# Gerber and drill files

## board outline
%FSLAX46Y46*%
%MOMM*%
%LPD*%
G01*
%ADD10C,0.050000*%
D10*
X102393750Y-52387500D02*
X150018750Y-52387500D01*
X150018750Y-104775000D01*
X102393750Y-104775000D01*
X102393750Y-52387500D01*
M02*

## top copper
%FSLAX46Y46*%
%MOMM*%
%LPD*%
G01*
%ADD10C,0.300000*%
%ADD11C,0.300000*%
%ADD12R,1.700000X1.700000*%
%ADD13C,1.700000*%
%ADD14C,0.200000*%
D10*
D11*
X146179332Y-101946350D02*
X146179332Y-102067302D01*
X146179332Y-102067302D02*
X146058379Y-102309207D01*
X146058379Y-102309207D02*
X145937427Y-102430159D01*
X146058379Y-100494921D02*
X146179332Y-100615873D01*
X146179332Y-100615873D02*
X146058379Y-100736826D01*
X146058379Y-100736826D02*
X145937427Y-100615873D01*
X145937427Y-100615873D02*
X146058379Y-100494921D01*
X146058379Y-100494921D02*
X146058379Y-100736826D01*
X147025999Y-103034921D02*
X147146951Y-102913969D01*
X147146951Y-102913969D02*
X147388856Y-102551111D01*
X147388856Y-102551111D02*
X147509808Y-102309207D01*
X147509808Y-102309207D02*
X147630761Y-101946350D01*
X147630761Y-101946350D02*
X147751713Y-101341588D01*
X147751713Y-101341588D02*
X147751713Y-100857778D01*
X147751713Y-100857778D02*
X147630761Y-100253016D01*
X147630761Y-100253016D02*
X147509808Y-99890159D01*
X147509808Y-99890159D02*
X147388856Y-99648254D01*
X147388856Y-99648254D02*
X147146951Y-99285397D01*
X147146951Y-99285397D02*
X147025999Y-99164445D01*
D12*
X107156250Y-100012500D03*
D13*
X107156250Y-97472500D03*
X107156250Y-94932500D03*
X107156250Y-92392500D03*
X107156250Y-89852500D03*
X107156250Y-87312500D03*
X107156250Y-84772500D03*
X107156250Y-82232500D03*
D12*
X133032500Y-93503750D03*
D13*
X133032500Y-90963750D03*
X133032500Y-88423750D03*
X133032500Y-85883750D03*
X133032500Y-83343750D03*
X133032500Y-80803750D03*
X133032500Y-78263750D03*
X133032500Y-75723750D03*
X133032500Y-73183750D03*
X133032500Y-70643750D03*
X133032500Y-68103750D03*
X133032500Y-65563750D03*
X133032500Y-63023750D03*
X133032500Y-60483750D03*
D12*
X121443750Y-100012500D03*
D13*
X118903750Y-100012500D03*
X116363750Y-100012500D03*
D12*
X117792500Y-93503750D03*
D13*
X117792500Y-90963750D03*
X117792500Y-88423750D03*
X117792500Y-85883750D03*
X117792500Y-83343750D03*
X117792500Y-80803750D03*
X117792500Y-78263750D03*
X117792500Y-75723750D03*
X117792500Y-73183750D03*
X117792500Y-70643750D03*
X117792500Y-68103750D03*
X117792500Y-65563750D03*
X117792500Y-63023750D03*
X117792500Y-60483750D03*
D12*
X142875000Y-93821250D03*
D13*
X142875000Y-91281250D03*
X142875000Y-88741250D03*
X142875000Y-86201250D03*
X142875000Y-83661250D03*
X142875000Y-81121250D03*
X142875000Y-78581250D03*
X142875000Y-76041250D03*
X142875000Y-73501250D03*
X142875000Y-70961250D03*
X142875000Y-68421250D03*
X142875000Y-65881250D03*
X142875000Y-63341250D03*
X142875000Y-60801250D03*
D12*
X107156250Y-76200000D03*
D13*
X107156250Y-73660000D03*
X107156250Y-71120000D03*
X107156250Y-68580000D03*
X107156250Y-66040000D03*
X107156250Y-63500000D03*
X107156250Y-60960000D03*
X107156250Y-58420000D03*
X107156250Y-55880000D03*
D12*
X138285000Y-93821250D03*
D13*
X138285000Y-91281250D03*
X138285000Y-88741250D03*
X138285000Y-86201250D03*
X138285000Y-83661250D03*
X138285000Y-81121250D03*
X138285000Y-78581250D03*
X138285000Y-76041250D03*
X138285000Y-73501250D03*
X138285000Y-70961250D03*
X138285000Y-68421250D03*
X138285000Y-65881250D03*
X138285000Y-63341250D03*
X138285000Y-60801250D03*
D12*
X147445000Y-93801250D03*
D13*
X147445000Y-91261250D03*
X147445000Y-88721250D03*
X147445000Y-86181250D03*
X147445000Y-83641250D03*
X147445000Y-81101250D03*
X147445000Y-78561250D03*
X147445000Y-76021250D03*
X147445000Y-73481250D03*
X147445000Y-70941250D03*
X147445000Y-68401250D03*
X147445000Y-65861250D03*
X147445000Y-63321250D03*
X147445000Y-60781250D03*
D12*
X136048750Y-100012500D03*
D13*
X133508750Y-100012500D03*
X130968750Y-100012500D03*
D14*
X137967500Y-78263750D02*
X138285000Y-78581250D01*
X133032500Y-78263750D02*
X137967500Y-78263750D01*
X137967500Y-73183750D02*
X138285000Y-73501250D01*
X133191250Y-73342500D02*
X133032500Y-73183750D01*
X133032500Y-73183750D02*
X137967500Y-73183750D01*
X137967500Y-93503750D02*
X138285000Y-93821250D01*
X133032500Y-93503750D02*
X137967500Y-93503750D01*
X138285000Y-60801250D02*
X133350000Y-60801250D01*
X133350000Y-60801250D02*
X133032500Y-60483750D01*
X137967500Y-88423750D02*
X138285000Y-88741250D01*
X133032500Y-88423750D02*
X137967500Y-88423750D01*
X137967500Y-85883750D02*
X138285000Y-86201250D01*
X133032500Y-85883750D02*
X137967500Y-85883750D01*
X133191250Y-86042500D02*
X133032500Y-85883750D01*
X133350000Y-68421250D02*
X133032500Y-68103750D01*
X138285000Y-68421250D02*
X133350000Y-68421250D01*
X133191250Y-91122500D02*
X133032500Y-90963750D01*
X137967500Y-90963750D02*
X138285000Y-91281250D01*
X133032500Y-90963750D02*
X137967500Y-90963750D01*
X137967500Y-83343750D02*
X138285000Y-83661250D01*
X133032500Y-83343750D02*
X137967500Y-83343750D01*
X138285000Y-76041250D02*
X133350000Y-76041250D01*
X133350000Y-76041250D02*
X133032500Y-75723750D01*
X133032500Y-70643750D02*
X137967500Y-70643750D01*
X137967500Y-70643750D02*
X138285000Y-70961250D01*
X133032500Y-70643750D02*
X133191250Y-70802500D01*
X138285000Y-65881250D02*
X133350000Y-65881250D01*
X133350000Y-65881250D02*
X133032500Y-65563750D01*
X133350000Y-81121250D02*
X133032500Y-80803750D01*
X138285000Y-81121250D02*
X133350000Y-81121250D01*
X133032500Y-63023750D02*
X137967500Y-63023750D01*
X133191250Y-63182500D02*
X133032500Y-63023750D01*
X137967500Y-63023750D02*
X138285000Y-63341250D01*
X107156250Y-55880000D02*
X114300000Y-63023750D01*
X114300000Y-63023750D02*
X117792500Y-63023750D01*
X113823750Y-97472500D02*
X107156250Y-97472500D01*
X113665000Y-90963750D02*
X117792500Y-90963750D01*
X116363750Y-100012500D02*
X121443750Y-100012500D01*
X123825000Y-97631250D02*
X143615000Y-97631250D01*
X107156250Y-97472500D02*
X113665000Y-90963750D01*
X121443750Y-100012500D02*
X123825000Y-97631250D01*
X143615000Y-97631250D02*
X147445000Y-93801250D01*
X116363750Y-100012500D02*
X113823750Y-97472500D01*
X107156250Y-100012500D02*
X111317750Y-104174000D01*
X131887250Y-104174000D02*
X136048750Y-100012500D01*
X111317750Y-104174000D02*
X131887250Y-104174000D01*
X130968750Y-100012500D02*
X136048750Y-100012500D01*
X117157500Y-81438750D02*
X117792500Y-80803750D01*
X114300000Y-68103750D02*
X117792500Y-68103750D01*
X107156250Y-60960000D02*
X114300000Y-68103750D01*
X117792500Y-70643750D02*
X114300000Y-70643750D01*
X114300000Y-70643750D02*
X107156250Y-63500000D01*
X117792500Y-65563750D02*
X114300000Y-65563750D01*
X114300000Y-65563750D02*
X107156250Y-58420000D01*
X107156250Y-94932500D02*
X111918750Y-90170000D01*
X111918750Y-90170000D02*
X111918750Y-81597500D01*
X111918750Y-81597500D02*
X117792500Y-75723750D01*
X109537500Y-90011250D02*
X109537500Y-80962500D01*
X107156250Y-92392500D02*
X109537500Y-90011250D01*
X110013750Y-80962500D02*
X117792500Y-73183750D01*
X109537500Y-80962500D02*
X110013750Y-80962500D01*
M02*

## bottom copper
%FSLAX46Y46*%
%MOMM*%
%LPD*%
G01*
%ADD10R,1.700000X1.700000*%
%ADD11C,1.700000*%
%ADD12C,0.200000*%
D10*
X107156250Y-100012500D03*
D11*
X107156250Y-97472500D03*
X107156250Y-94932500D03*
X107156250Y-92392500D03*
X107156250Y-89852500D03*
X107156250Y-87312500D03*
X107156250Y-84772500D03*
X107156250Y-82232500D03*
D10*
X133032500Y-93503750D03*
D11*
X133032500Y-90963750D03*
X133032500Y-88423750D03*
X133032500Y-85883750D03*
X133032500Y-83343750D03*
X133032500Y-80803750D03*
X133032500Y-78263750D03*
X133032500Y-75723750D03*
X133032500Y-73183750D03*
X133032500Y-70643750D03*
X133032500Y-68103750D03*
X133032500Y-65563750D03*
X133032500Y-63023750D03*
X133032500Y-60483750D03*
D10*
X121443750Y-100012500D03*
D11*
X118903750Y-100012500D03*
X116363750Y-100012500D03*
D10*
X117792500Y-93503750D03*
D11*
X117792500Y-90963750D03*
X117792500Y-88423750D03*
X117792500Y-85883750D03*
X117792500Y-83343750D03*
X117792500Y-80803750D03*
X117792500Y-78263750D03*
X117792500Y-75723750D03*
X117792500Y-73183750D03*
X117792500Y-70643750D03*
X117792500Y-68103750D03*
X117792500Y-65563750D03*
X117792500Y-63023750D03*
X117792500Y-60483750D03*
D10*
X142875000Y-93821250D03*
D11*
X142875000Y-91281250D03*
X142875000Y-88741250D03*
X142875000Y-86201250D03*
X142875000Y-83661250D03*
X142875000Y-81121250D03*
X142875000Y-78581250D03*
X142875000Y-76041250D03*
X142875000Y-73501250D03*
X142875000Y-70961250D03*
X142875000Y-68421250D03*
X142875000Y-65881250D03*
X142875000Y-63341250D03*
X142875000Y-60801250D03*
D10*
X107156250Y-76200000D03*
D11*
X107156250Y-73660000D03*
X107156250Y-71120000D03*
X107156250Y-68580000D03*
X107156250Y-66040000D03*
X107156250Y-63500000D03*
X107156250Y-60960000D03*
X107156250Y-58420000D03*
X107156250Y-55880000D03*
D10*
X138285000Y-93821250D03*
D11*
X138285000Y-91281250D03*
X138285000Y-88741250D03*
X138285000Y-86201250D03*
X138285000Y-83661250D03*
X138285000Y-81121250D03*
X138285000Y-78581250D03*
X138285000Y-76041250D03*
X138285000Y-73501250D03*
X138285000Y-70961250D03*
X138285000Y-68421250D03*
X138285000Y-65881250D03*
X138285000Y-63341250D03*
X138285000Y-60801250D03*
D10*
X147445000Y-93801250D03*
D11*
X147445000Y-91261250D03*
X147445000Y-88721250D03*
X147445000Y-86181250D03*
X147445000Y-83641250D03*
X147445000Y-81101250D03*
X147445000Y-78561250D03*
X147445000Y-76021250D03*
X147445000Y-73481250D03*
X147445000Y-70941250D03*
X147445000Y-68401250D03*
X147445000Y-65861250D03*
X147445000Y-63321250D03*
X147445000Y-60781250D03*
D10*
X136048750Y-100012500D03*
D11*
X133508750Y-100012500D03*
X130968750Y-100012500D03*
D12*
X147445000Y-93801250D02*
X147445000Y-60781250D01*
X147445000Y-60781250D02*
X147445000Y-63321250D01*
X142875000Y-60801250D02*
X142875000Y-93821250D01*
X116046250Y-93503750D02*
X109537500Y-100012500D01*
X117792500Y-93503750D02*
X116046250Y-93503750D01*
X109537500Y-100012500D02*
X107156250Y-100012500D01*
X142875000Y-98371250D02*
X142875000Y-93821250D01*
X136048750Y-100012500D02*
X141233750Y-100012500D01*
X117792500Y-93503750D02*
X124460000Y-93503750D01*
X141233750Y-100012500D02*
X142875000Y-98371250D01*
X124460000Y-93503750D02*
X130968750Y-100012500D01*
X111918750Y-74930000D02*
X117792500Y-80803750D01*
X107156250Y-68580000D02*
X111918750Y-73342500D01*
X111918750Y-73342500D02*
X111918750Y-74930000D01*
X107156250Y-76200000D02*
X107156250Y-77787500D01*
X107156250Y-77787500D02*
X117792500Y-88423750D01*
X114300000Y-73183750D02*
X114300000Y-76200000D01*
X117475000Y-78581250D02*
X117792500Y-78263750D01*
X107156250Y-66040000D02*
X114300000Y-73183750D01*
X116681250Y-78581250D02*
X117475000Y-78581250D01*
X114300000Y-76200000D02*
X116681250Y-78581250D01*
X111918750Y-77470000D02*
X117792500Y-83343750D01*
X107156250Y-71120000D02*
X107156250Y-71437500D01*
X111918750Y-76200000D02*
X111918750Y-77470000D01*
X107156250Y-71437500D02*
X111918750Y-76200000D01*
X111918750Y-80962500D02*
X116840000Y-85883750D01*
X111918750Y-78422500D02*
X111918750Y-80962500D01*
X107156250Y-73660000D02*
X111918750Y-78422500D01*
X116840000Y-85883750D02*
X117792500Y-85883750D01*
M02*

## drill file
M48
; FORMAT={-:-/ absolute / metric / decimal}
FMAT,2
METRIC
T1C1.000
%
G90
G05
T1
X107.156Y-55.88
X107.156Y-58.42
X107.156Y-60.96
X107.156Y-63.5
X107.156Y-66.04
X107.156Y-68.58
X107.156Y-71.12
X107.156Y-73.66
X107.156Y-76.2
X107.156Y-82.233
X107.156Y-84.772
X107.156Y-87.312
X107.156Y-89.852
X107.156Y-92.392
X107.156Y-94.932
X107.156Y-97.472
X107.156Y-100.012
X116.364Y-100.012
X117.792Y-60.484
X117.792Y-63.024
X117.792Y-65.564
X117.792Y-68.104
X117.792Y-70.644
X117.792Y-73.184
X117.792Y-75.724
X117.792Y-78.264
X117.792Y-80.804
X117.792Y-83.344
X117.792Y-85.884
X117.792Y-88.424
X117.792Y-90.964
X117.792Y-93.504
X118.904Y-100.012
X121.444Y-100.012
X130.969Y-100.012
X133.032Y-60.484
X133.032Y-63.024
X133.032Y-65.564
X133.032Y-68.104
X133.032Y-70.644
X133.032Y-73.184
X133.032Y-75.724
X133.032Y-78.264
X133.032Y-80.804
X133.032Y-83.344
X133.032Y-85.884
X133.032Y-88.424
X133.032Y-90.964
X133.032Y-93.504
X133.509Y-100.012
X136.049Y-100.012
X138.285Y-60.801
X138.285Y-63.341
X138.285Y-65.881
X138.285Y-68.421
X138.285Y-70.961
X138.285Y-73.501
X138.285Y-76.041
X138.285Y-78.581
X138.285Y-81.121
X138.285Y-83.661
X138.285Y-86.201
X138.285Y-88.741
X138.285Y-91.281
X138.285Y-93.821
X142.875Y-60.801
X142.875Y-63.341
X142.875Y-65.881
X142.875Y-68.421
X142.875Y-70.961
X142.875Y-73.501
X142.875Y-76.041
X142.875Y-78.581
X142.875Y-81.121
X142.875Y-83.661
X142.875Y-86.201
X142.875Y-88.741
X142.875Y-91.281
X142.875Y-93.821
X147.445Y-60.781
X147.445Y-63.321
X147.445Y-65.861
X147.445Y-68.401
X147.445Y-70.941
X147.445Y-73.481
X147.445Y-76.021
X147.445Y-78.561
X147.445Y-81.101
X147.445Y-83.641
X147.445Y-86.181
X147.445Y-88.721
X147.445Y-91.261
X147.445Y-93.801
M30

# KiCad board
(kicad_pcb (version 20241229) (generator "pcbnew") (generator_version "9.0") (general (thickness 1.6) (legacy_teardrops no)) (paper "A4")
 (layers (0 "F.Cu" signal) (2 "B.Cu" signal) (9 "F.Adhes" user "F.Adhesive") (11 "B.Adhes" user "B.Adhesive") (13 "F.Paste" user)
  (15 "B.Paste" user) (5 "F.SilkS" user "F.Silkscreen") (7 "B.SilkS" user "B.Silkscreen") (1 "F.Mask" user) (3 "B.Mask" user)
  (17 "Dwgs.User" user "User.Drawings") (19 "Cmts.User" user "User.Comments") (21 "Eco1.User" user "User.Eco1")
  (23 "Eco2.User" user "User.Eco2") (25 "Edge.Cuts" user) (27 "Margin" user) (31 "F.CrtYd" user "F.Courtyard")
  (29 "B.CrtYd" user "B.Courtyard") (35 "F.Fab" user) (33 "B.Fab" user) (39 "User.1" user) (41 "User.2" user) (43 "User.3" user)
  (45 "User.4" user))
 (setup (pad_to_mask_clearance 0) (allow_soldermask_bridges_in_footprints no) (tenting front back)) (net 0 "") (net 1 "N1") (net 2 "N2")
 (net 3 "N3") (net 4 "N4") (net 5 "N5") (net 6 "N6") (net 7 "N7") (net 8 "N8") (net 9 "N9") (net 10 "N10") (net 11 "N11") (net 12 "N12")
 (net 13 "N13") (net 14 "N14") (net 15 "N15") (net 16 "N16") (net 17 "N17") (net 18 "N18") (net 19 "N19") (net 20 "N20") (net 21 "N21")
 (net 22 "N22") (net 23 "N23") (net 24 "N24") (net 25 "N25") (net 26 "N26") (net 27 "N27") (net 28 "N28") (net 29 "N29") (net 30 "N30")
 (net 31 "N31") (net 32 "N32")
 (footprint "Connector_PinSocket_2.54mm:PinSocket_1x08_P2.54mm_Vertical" (layer "F.Cu") (at 107.15625 100.0125 180)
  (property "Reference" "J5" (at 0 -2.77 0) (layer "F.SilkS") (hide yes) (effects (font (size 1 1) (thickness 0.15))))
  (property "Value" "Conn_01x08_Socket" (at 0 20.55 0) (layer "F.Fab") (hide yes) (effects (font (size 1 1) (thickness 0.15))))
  (pad "1" thru_hole rect (at 0 0 180) (size 1.7 1.7) (drill 1) (layers "*.Cu" "*.Mask") (remove_unused_layers no) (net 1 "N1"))
  (pad "2" thru_hole circle (at 0 2.54 180) (size 1.7 1.7) (drill 1) (layers "*.Cu" "*.Mask") (remove_unused_layers no) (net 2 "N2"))
  (pad "3" thru_hole circle (at 0 5.08 180) (size 1.7 1.7) (drill 1) (layers "*.Cu" "*.Mask") (remove_unused_layers no) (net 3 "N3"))
  (pad "4" thru_hole circle (at 0 7.62 180) (size 1.7 1.7) (drill 1) (layers "*.Cu" "*.Mask") (remove_unused_layers no) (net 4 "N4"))
  (pad "5" thru_hole circle (at 0 10.16 180) (size 1.7 1.7) (drill 1) (layers "*.Cu" "*.Mask") (remove_unused_layers no) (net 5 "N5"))
  (pad "6" thru_hole circle (at 0 12.7 180) (size 1.7 1.7) (drill 1) (layers "*.Cu" "*.Mask") (remove_unused_layers no) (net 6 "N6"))
  (pad "7" thru_hole circle (at 0 15.24 180) (size 1.7 1.7) (drill 1) (layers "*.Cu" "*.Mask") (remove_unused_layers no) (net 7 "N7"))
  (pad "8" thru_hole circle (at 0 17.78 180) (size 1.7 1.7) (drill 1) (layers "*.Cu" "*.Mask") (remove_unused_layers no) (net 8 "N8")))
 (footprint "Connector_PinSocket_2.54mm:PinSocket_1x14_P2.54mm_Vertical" (layer "F.Cu") (at 133.0325 93.50375 180)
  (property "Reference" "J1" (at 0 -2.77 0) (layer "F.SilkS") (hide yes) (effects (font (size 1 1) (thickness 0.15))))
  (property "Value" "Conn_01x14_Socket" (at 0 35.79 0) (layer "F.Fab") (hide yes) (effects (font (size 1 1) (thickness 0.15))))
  (pad "1" thru_hole rect (at 0 0 180) (size 1.7 1.7) (drill 1) (layers "*.Cu" "*.Mask") (remove_unused_layers no) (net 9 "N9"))
  (pad "2" thru_hole circle (at 0 2.54 180) (size 1.7 1.7) (drill 1) (layers "*.Cu" "*.Mask") (remove_unused_layers no) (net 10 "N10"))
  (pad "3" thru_hole circle (at 0 5.08 180) (size 1.7 1.7) (drill 1) (layers "*.Cu" "*.Mask") (remove_unused_layers no) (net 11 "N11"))
  (pad "4" thru_hole circle (at 0 7.62 180) (size 1.7 1.7) (drill 1) (layers "*.Cu" "*.Mask") (remove_unused_layers no) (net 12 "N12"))
  (pad "5" thru_hole circle (at 0 10.16 180) (size 1.7 1.7) (drill 1) (layers "*.Cu" "*.Mask") (remove_unused_layers no) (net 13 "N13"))
  (pad "6" thru_hole circle (at 0 12.7 180) (size 1.7 1.7) (drill 1) (layers "*.Cu" "*.Mask") (remove_unused_layers no) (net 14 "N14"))
  (pad "7" thru_hole circle (at 0 15.24 180) (size 1.7 1.7) (drill 1) (layers "*.Cu" "*.Mask") (remove_unused_layers no) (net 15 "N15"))
  (pad "8" thru_hole circle (at 0 17.78 180) (size 1.7 1.7) (drill 1) (layers "*.Cu" "*.Mask") (remove_unused_layers no) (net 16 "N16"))
  (pad "9" thru_hole circle (at 0 20.32 180) (size 1.7 1.7) (drill 1) (layers "*.Cu" "*.Mask") (remove_unused_layers no) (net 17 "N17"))
  (pad "10" thru_hole circle (at 0 22.86 180) (size 1.7 1.7) (drill 1) (layers "*.Cu" "*.Mask") (remove_unused_layers no) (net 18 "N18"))
  (pad "11" thru_hole circle (at 0 25.4 180) (size 1.7 1.7) (drill 1) (layers "*.Cu" "*.Mask") (remove_unused_layers no) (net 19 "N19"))
  (pad "12" thru_hole circle (at 0 27.94 180) (size 1.7 1.7) (drill 1) (layers "*.Cu" "*.Mask") (remove_unused_layers no) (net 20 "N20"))
  (pad "13" thru_hole circle (at 0 30.48 180) (size 1.7 1.7) (drill 1) (layers "*.Cu" "*.Mask") (remove_unused_layers no) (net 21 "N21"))
  (pad "14" thru_hole circle (at 0 33.02 180) (size 1.7 1.7) (drill 1) (layers "*.Cu" "*.Mask") (remove_unused_layers no) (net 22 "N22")))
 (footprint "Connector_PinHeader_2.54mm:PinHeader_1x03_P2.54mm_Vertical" (layer "F.Cu") (at 121.44375 100.0125 -90)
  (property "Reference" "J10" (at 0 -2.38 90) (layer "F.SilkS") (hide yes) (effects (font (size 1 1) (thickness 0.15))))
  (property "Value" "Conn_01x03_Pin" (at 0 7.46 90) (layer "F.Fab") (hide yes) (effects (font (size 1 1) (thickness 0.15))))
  (pad "1" thru_hole rect (at 0 0 270) (size 1.7 1.7) (drill 1) (layers "*.Cu" "*.Mask") (remove_unused_layers no) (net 2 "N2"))
  (pad "2" thru_hole circle (at 0 2.54 270) (size 1.7 1.7) (drill 1) (layers "*.Cu" "*.Mask") (remove_unused_layers no) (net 2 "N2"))
  (pad "3" thru_hole circle (at 0 5.08 270) (size 1.7 1.7) (drill 1) (layers "*.Cu" "*.Mask") (remove_unused_layers no) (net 2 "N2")))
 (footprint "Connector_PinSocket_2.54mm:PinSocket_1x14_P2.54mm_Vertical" (layer "F.Cu") (at 117.7925 93.50375 180)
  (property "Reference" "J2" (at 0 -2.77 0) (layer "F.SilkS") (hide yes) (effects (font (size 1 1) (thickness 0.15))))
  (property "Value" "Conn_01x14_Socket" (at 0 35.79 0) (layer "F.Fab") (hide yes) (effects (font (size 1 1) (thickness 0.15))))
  (pad "1" thru_hole rect (at 0 0 180) (size 1.7 1.7) (drill 1) (layers "*.Cu" "*.Mask") (remove_unused_layers no) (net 1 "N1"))
  (pad "2" thru_hole circle (at 0 2.54 180) (size 1.7 1.7) (drill 1) (layers "*.Cu" "*.Mask") (remove_unused_layers no) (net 2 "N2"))
  (pad "3" thru_hole circle (at 0 5.08 180) (size 1.7 1.7) (drill 1) (layers "*.Cu" "*.Mask") (remove_unused_layers no) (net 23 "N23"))
  (pad "4" thru_hole circle (at 0 7.62 180) (size 1.7 1.7) (drill 1) (layers "*.Cu" "*.Mask") (remove_unused_layers no) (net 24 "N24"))
  (pad "5" thru_hole circle (at 0 10.16 180) (size 1.7 1.7) (drill 1) (layers "*.Cu" "*.Mask") (remove_unused_layers no) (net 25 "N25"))
  (pad "6" thru_hole circle (at 0 12.7 180) (size 1.7 1.7) (drill 1) (layers "*.Cu" "*.Mask") (remove_unused_layers no) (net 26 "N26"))
  (pad "7" thru_hole circle (at 0 15.24 180) (size 1.7 1.7) (drill 1) (layers "*.Cu" "*.Mask") (remove_unused_layers no) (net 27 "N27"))
  (pad "8" thru_hole circle (at 0 17.78 180) (size 1.7 1.7) (drill 1) (layers "*.Cu" "*.Mask") (remove_unused_layers no) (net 3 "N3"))
  (pad "9" thru_hole circle (at 0 20.32 180) (size 1.7 1.7) (drill 1) (layers "*.Cu" "*.Mask") (remove_unused_layers no) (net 4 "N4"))
  (pad "10" thru_hole circle (at 0 22.86 180) (size 1.7 1.7) (drill 1) (layers "*.Cu" "*.Mask") (remove_unused_layers no) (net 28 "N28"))
  (pad "11" thru_hole circle (at 0 25.4 180) (size 1.7 1.7) (drill 1) (layers "*.Cu" "*.Mask") (remove_unused_layers no) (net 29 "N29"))
  (pad "12" thru_hole circle (at 0 27.94 180) (size 1.7 1.7) (drill 1) (layers "*.Cu" "*.Mask") (remove_unused_layers no) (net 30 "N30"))
  (pad "13" thru_hole circle (at 0 30.48 180) (size 1.7 1.7) (drill 1) (layers "*.Cu" "*.Mask") (remove_unused_layers no) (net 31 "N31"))
  (pad "14" thru_hole circle (at 0 33.02 180) (size 1.7 1.7) (drill 1) (layers "*.Cu" "*.Mask") (remove_unused_layers no) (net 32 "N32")))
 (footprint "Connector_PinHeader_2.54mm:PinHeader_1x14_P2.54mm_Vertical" (layer "F.Cu") (at 142.875 93.82125 180)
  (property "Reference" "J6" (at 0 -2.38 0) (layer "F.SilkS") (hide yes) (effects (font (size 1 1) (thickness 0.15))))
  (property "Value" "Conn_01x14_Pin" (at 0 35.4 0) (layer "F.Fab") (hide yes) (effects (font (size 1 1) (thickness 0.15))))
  (pad "1" thru_hole rect (at 0 0 180) (size 1.7 1.7) (drill 1) (layers "*.Cu" "*.Mask") (remove_unused_layers no) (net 1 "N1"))
  (pad "2" thru_hole circle (at 0 2.54 180) (size 1.7 1.7) (drill 1) (layers "*.Cu" "*.Mask") (remove_unused_layers no) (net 1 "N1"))
  (pad "3" thru_hole circle (at 0 5.08 180) (size 1.7 1.7) (drill 1) (layers "*.Cu" "*.Mask") (remove_unused_layers no) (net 1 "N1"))
  (pad "4" thru_hole circle (at 0 7.62 180) (size 1.7 1.7) (drill 1) (layers "*.Cu" "*.Mask") (remove_unused_layers no) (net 1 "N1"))
  (pad "5" thru_hole circle (at 0 10.16 180) (size 1.7 1.7) (drill 1) (layers "*.Cu" "*.Mask") (remove_unused_layers no) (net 1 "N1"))
  (pad "6" thru_hole circle (at 0 12.7 180) (size 1.7 1.7) (drill 1) (layers "*.Cu" "*.Mask") (remove_unused_layers no) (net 1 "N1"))
  (pad "7" thru_hole circle (at 0 15.24 180) (size 1.7 1.7) (drill 1) (layers "*.Cu" "*.Mask") (remove_unused_layers no) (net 1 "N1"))
  (pad "8" thru_hole circle (at 0 17.78 180) (size 1.7 1.7) (drill 1) (layers "*.Cu" "*.Mask") (remove_unused_layers no) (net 1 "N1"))
  (pad "9" thru_hole circle (at 0 20.32 180) (size 1.7 1.7) (drill 1) (layers "*.Cu" "*.Mask") (remove_unused_layers no) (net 1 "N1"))
  (pad "10" thru_hole circle (at 0 22.86 180) (size 1.7 1.7) (drill 1) (layers "*.Cu" "*.Mask") (remove_unused_layers no) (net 1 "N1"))
  (pad "11" thru_hole circle (at 0 25.4 180) (size 1.7 1.7) (drill 1) (layers "*.Cu" "*.Mask") (remove_unused_layers no) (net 1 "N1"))
  (pad "12" thru_hole circle (at 0 27.94 180) (size 1.7 1.7) (drill 1) (layers "*.Cu" "*.Mask") (remove_unused_layers no) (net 1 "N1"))
  (pad "13" thru_hole circle (at 0 30.48 180) (size 1.7 1.7) (drill 1) (layers "*.Cu" "*.Mask") (remove_unused_layers no) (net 1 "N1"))
  (pad "14" thru_hole circle (at 0 33.02 180) (size 1.7 1.7) (drill 1) (layers "*.Cu" "*.Mask") (remove_unused_layers no) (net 1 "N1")))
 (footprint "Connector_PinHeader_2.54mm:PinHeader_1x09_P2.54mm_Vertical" (layer "F.Cu") (at 107.15625 76.2 180)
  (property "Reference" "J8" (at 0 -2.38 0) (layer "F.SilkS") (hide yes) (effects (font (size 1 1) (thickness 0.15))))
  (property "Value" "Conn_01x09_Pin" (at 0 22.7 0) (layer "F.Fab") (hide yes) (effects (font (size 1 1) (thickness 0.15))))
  (pad "1" thru_hole rect (at 0 0 180) (size 1.7 1.7) (drill 1) (layers "*.Cu" "*.Mask") (remove_unused_layers no) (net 23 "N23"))
  (pad "2" thru_hole circle (at 0 2.54 180) (size 1.7 1.7) (drill 1) (layers "*.Cu" "*.Mask") (remove_unused_layers no) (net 24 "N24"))
  (pad "3" thru_hole circle (at 0 5.08 180) (size 1.7 1.7) (drill 1) (layers "*.Cu" "*.Mask") (remove_unused_layers no) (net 25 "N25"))
  (pad "4" thru_hole circle (at 0 7.62 180) (size 1.7 1.7) (drill 1) (layers "*.Cu" "*.Mask") (remove_unused_layers no) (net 26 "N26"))
  (pad "5" thru_hole circle (at 0 10.16 180) (size 1.7 1.7) (drill 1) (layers "*.Cu" "*.Mask") (remove_unused_layers no) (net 27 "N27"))
  (pad "6" thru_hole circle (at 0 12.7 180) (size 1.7 1.7) (drill 1) (layers "*.Cu" "*.Mask") (remove_unused_layers no) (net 28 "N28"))
  (pad "7" thru_hole circle (at 0 15.24 180) (size 1.7 1.7) (drill 1) (layers "*.Cu" "*.Mask") (remove_unused_layers no) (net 29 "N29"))
  (pad "8" thru_hole circle (at 0 17.78 180) (size 1.7 1.7) (drill 1) (layers "*.Cu" "*.Mask") (remove_unused_layers no) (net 30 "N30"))
  (pad "9" thru_hole circle (at 0 20.32 180) (size 1.7 1.7) (drill 1) (layers "*.Cu" "*.Mask") (remove_unused_layers no) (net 31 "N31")))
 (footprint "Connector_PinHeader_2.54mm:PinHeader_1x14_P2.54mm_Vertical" (layer "F.Cu") (at 138.285 93.82125 180)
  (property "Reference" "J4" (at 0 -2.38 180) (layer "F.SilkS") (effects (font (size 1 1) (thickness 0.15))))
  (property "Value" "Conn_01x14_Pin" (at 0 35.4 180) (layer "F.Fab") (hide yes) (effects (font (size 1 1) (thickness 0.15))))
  (pad "1" thru_hole rect (at 0 0 180) (size 1.7 1.7) (drill 1) (layers "*.Cu" "*.Mask") (remove_unused_layers no) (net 9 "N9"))
  (pad "2" thru_hole circle (at 0 2.54 180) (size 1.7 1.7) (drill 1) (layers "*.Cu" "*.Mask") (remove_unused_layers no) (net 10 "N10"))
  (pad "3" thru_hole circle (at 0 5.08 180) (size 1.7 1.7) (drill 1) (layers "*.Cu" "*.Mask") (remove_unused_layers no) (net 11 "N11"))
  (pad "4" thru_hole circle (at 0 7.62 180) (size 1.7 1.7) (drill 1) (layers "*.Cu" "*.Mask") (remove_unused_layers no) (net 12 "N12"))
  (pad "5" thru_hole circle (at 0 10.16 180) (size 1.7 1.7) (drill 1) (layers "*.Cu" "*.Mask") (remove_unused_layers no) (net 13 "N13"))
  (pad "6" thru_hole circle (at 0 12.7 180) (size 1.7 1.7) (drill 1) (layers "*.Cu" "*.Mask") (remove_unused_layers no) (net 14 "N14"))
  (pad "7" thru_hole circle (at 0 15.24 180) (size 1.7 1.7) (drill 1) (layers "*.Cu" "*.Mask") (remove_unused_layers no) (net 15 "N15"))
  (pad "8" thru_hole circle (at 0 17.78 180) (size 1.7 1.7) (drill 1) (layers "*.Cu" "*.Mask") (remove_unused_layers no) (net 16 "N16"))
  (pad "9" thru_hole circle (at 0 20.32 180) (size 1.7 1.7) (drill 1) (layers "*.Cu" "*.Mask") (remove_unused_layers no) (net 17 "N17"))
  (pad "10" thru_hole circle (at 0 22.86 180) (size 1.7 1.7) (drill 1) (layers "*.Cu" "*.Mask") (remove_unused_layers no) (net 18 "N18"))
  (pad "11" thru_hole circle (at 0 25.4 180) (size 1.7 1.7) (drill 1) (layers "*.Cu" "*.Mask") (remove_unused_layers no) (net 19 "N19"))
  (pad "12" thru_hole circle (at 0 27.94 180) (size 1.7 1.7) (drill 1) (layers "*.Cu" "*.Mask") (remove_unused_layers no) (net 20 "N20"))
  (pad "13" thru_hole circle (at 0 30.48 180) (size 1.7 1.7) (drill 1) (layers "*.Cu" "*.Mask") (remove_unused_layers no) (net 21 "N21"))
  (pad "14" thru_hole circle (at 0 33.02 180) (size 1.7 1.7) (drill 1) (layers "*.Cu" "*.Mask") (remove_unused_layers no) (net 22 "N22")))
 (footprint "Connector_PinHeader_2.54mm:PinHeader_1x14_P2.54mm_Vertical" (layer "F.Cu") (at 147.445 93.80125 180)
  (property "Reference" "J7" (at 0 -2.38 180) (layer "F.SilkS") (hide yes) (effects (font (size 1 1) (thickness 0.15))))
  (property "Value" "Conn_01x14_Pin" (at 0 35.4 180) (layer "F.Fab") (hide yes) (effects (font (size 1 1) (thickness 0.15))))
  (pad "1" thru_hole rect (at 0 0 180) (size 1.7 1.7) (drill 1) (layers "*.Cu" "*.Mask") (remove_unused_layers no) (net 2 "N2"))
  (pad "2" thru_hole circle (at 0 2.54 180) (size 1.7 1.7) (drill 1) (layers "*.Cu" "*.Mask") (remove_unused_layers no) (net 2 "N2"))
  (pad "3" thru_hole circle (at 0 5.08 180) (size 1.7 1.7) (drill 1) (layers "*.Cu" "*.Mask") (remove_unused_layers no) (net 2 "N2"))
  (pad "4" thru_hole circle (at 0 7.62 180) (size 1.7 1.7) (drill 1) (layers "*.Cu" "*.Mask") (remove_unused_layers no) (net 2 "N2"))
  (pad "5" thru_hole circle (at 0 10.16 180) (size 1.7 1.7) (drill 1) (layers "*.Cu" "*.Mask") (remove_unused_layers no) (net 2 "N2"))
  (pad "6" thru_hole circle (at 0 12.7 180) (size 1.7 1.7) (drill 1) (layers "*.Cu" "*.Mask") (remove_unused_layers no) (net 2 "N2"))
  (pad "7" thru_hole circle (at 0 15.24 180) (size 1.7 1.7) (drill 1) (layers "*.Cu" "*.Mask") (remove_unused_layers no) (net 2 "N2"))
  (pad "8" thru_hole circle (at 0 17.78 180) (size 1.7 1.7) (drill 1) (layers "*.Cu" "*.Mask") (remove_unused_layers no) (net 2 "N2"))
  (pad "9" thru_hole circle (at 0 20.32 180) (size 1.7 1.7) (drill 1) (layers "*.Cu" "*.Mask") (remove_unused_layers no) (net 2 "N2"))
  (pad "10" thru_hole circle (at 0 22.86 180) (size 1.7 1.7) (drill 1) (layers "*.Cu" "*.Mask") (remove_unused_layers no) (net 2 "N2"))
  (pad "11" thru_hole circle (at 0 25.4 180) (size 1.7 1.7) (drill 1) (layers "*.Cu" "*.Mask") (remove_unused_layers no) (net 2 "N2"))
  (pad "12" thru_hole circle (at 0 27.94 180) (size 1.7 1.7) (drill 1) (layers "*.Cu" "*.Mask") (remove_unused_layers no) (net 2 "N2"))
  (pad "13" thru_hole circle (at 0 30.48 180) (size 1.7 1.7) (drill 1) (layers "*.Cu" "*.Mask") (remove_unused_layers no) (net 2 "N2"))
  (pad "14" thru_hole circle (at 0 33.02 180) (size 1.7 1.7) (drill 1) (layers "*.Cu" "*.Mask") (remove_unused_layers no) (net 2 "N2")))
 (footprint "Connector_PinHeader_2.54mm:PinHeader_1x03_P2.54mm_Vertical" (layer "F.Cu") (at 136.04875 100.0125 -90)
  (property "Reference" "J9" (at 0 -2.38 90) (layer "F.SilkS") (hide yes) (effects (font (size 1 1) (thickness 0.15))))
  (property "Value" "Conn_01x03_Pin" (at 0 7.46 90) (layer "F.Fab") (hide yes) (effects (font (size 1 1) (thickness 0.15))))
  (pad "1" thru_hole rect (at 0 0 270) (size 1.7 1.7) (drill 1) (layers "*.Cu" "*.Mask") (remove_unused_layers no) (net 1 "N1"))
  (pad "2" thru_hole circle (at 0 2.54 270) (size 1.7 1.7) (drill 1) (layers "*.Cu" "*.Mask") (remove_unused_layers no) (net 1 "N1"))
  (pad "3" thru_hole circle (at 0 5.08 270) (size 1.7 1.7) (drill 1) (layers "*.Cu" "*.Mask") (remove_unused_layers no) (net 1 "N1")))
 (gr_rect (start 102.39375 52.3875) (end 150.01875 104.775) (stroke (width 0.05) (type default)) (fill no) (layer "Edge.Cuts"))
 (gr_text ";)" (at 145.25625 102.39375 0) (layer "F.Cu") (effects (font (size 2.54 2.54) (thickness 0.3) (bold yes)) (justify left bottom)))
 (segment (start 137.9675 78.26375) (end 138.285 78.58125) (width 0.2) (layer "F.Cu") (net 15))
 (segment (start 133.0325 78.26375) (end 137.9675 78.26375) (width 0.2) (layer "F.Cu") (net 15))
 (segment (start 137.9675 73.18375) (end 138.285 73.50125) (width 0.2) (layer "F.Cu") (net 17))
 (segment (start 133.19125 73.3425) (end 133.0325 73.18375) (width 0.2) (layer "F.Cu") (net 17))
 (segment (start 133.0325 73.18375) (end 137.9675 73.18375) (width 0.2) (layer "F.Cu") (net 17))
 (segment (start 137.9675 93.50375) (end 138.285 93.82125) (width 0.2) (layer "F.Cu") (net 9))
 (segment (start 133.0325 93.50375) (end 137.9675 93.50375) (width 0.2) (layer "F.Cu") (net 9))
 (segment (start 138.285 60.80125) (end 133.35 60.80125) (width 0.2) (layer "F.Cu") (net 22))
 (segment (start 133.35 60.80125) (end 133.0325 60.48375) (width 0.2) (layer "F.Cu") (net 22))
 (segment (start 137.9675 88.42375) (end 138.285 88.74125) (width 0.2) (layer "F.Cu") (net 11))
 (segment (start 133.0325 88.42375) (end 137.9675 88.42375) (width 0.2) (layer "F.Cu") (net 11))
 (segment (start 137.9675 85.88375) (end 138.285 86.20125) (width 0.2) (layer "F.Cu") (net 12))
 (segment (start 133.0325 85.88375) (end 137.9675 85.88375) (width 0.2) (layer "F.Cu") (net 12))
 (segment (start 133.19125 86.0425) (end 133.0325 85.88375) (width 0.2) (layer "F.Cu") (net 12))
 (segment (start 133.35 68.42125) (end 133.0325 68.10375) (width 0.2) (layer "F.Cu") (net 19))
 (segment (start 138.285 68.42125) (end 133.35 68.42125) (width 0.2) (layer "F.Cu") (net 19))
 (segment (start 133.19125 91.1225) (end 133.0325 90.96375) (width 0.2) (layer "F.Cu") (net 10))
 (segment (start 137.9675 90.96375) (end 138.285 91.28125) (width 0.2) (layer "F.Cu") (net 10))
 (segment (start 133.0325 90.96375) (end 137.9675 90.96375) (width 0.2) (layer "F.Cu") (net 10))
 (segment (start 137.9675 83.34375) (end 138.285 83.66125) (width 0.2) (layer "F.Cu") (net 13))
 (segment (start 133.0325 83.34375) (end 137.9675 83.34375) (width 0.2) (layer "F.Cu") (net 13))
 (segment (start 138.285 76.04125) (end 133.35 76.04125) (width 0.2) (layer "F.Cu") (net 16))
 (segment (start 133.35 76.04125) (end 133.0325 75.72375) (width 0.2) (layer "F.Cu") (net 16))
 (segment (start 133.0325 70.64375) (end 137.9675 70.64375) (width 0.2) (layer "F.Cu") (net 18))
 (segment (start 137.9675 70.64375) (end 138.285 70.96125) (width 0.2) (layer "F.Cu") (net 18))
 (segment (start 133.0325 70.64375) (end 133.19125 70.8025) (width 0.2) (layer "F.Cu") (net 18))
 (segment (start 138.285 65.88125) (end 133.35 65.88125) (width 0.2) (layer "F.Cu") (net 20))
 (segment (start 133.35 65.88125) (end 133.0325 65.56375) (width 0.2) (layer "F.Cu") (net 20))
 (segment (start 133.35 81.12125) (end 133.0325 80.80375) (width 0.2) (layer "F.Cu") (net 14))
 (segment (start 138.285 81.12125) (end 133.35 81.12125) (width 0.2) (layer "F.Cu") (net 14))
 (segment (start 133.0325 63.02375) (end 137.9675 63.02375) (width 0.2) (layer "F.Cu") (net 21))
 (segment (start 133.19125 63.1825) (end 133.0325 63.02375) (width 0.2) (layer "F.Cu") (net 21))
 (segment (start 137.9675 63.02375) (end 138.285 63.34125) (width 0.2) (layer "F.Cu") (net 21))
 (segment (start 107.15625 55.88) (end 114.3 63.02375) (width 0.2) (layer "F.Cu") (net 31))
 (segment (start 114.3 63.02375) (end 117.7925 63.02375) (width 0.2) (layer "F.Cu") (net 31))
 (segment (start 113.82375 97.4725) (end 107.15625 97.4725) (width 0.2) (layer "F.Cu") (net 2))
 (segment (start 113.665 90.96375) (end 117.7925 90.96375) (width 0.2) (layer "F.Cu") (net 2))
 (segment (start 116.36375 100.0125) (end 121.44375 100.0125) (width 0.2) (layer "F.Cu") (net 2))
 (segment (start 123.825 97.63125) (end 143.615 97.63125) (width 0.2) (layer "F.Cu") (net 2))
 (segment (start 107.15625 97.4725) (end 113.665 90.96375) (width 0.2) (layer "F.Cu") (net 2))
 (segment (start 121.44375 100.0125) (end 123.825 97.63125) (width 0.2) (layer "F.Cu") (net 2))
 (segment (start 143.615 97.63125) (end 147.445 93.80125) (width 0.2) (layer "F.Cu") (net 2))
 (segment (start 116.36375 100.0125) (end 113.82375 97.4725) (width 0.2) (layer "F.Cu") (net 2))
 (segment (start 147.445 93.80125) (end 147.445 60.78125) (width 0.2) (layer "B.Cu") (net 2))
 (segment (start 147.445 60.78125) (end 147.445 63.32125) (width 0.2) (layer "B.Cu") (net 2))
 (segment (start 107.15625 100.0125) (end 111.31775 104.174) (width 0.2) (layer "F.Cu") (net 1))
 (segment (start 131.88725 104.174) (end 136.04875 100.0125) (width 0.2) (layer "F.Cu") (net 1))
 (segment (start 111.31775 104.174) (end 131.88725 104.174) (width 0.2) (layer "F.Cu") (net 1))
 (segment (start 130.96875 100.0125) (end 136.04875 100.0125) (width 0.2) (layer "F.Cu") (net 1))
 (segment (start 142.875 60.80125) (end 142.875 93.82125) (width 0.2) (layer "B.Cu") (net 1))
 (segment (start 116.04625 93.50375) (end 109.5375 100.0125) (width 0.2) (layer "B.Cu") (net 1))
 (segment (start 117.7925 93.50375) (end 116.04625 93.50375) (width 0.2) (layer "B.Cu") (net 1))
 (segment (start 109.5375 100.0125) (end 107.15625 100.0125) (width 0.2) (layer "B.Cu") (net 1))
 (segment (start 142.875 98.37125) (end 142.875 93.82125) (width 0.2) (layer "B.Cu") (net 1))
 (segment (start 136.04875 100.0125) (end 141.23375 100.0125) (width 0.2) (layer "B.Cu") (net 1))
 (segment (start 117.7925 93.50375) (end 124.46 93.50375) (width 0.2) (layer "B.Cu") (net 1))
 (segment (start 141.23375 100.0125) (end 142.875 98.37125) (width 0.2) (layer "B.Cu") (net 1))
 (segment (start 124.46 93.50375) (end 130.96875 100.0125) (width 0.2) (layer "B.Cu") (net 1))
 (segment (start 117.1575 81.43875) (end 117.7925 80.80375) (width 0.2) (layer "F.Cu") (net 26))
 (segment (start 111.91875 74.93) (end 117.7925 80.80375) (width 0.2) (layer "B.Cu") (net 26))
 (segment (start 107.15625 68.58) (end 111.91875 73.3425) (width 0.2) (layer "B.Cu") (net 26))
 (segment (start 111.91875 73.3425) (end 111.91875 74.93) (width 0.2) (layer "B.Cu") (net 26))
 (segment (start 114.3 68.10375) (end 117.7925 68.10375) (width 0.2) (layer "F.Cu") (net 29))
 (segment (start 107.15625 60.96) (end 114.3 68.10375) (width 0.2) (layer "F.Cu") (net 29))
 (segment (start 117.7925 70.64375) (end 114.3 70.64375) (width 0.2) (layer "F.Cu") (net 28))
 (segment (start 114.3 70.64375) (end 107.15625 63.5) (width 0.2) (layer "F.Cu") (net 28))
 (segment (start 107.15625 76.2) (end 107.15625 77.7875) (width 0.2) (layer "B.Cu") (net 23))
 (segment (start 107.15625 77.7875) (end 117.7925 88.42375) (width 0.2) (layer "B.Cu") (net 23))
 (segment (start 114.3 73.18375) (end 114.3 76.2) (width 0.2) (layer "B.Cu") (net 27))
 (segment (start 117.475 78.58125) (end 117.7925 78.26375) (width 0.2) (layer "B.Cu") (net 27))
 (segment (start 107.15625 66.04) (end 114.3 73.18375) (width 0.2) (layer "B.Cu") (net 27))
 (segment (start 116.68125 78.58125) (end 117.475 78.58125) (width 0.2) (layer "B.Cu") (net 27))
 (segment (start 114.3 76.2) (end 116.68125 78.58125) (width 0.2) (layer "B.Cu") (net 27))
 (segment (start 117.7925 65.56375) (end 114.3 65.56375) (width 0.2) (layer "F.Cu") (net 30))
 (segment (start 114.3 65.56375) (end 107.15625 58.42) (width 0.2) (layer "F.Cu") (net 30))
 (segment (start 111.91875 77.47) (end 117.7925 83.34375) (width 0.2) (layer "B.Cu") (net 25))
 (segment (start 107.15625 71.12) (end 107.15625 71.4375) (width 0.2) (layer "B.Cu") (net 25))
 (segment (start 111.91875 76.2) (end 111.91875 77.47) (width 0.2) (layer "B.Cu") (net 25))
 (segment (start 107.15625 71.4375) (end 111.91875 76.2) (width 0.2) (layer "B.Cu") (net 25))
 (segment (start 111.91875 80.9625) (end 116.84 85.88375) (width 0.2) (layer "B.Cu") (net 24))
 (segment (start 111.91875 78.4225) (end 111.91875 80.9625) (width 0.2) (layer "B.Cu") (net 24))
 (segment (start 107.15625 73.66) (end 111.91875 78.4225) (width 0.2) (layer "B.Cu") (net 24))
 (segment (start 116.84 85.88375) (end 117.7925 85.88375) (width 0.2) (layer "B.Cu") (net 24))
 (segment (start 107.15625 94.9325) (end 111.91875 90.17) (width 0.2) (layer "F.Cu") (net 3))
 (segment (start 111.91875 90.17) (end 111.91875 81.5975) (width 0.2) (layer "F.Cu") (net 3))
 (segment (start 111.91875 81.5975) (end 117.7925 75.72375) (width 0.2) (layer "F.Cu") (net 3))
 (segment (start 109.5375 90.01125) (end 109.5375 80.9625) (width 0.2) (layer "F.Cu") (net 4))
 (segment (start 107.15625 92.3925) (end 109.5375 90.01125) (width 0.2) (layer "F.Cu") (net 4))
 (segment (start 110.01375 80.9625) (end 117.7925 73.18375) (width 0.2) (layer "F.Cu") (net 4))
 (segment (start 109.5375 80.9625) (end 110.01375 80.9625) (width 0.2) (layer "F.Cu") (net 4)))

